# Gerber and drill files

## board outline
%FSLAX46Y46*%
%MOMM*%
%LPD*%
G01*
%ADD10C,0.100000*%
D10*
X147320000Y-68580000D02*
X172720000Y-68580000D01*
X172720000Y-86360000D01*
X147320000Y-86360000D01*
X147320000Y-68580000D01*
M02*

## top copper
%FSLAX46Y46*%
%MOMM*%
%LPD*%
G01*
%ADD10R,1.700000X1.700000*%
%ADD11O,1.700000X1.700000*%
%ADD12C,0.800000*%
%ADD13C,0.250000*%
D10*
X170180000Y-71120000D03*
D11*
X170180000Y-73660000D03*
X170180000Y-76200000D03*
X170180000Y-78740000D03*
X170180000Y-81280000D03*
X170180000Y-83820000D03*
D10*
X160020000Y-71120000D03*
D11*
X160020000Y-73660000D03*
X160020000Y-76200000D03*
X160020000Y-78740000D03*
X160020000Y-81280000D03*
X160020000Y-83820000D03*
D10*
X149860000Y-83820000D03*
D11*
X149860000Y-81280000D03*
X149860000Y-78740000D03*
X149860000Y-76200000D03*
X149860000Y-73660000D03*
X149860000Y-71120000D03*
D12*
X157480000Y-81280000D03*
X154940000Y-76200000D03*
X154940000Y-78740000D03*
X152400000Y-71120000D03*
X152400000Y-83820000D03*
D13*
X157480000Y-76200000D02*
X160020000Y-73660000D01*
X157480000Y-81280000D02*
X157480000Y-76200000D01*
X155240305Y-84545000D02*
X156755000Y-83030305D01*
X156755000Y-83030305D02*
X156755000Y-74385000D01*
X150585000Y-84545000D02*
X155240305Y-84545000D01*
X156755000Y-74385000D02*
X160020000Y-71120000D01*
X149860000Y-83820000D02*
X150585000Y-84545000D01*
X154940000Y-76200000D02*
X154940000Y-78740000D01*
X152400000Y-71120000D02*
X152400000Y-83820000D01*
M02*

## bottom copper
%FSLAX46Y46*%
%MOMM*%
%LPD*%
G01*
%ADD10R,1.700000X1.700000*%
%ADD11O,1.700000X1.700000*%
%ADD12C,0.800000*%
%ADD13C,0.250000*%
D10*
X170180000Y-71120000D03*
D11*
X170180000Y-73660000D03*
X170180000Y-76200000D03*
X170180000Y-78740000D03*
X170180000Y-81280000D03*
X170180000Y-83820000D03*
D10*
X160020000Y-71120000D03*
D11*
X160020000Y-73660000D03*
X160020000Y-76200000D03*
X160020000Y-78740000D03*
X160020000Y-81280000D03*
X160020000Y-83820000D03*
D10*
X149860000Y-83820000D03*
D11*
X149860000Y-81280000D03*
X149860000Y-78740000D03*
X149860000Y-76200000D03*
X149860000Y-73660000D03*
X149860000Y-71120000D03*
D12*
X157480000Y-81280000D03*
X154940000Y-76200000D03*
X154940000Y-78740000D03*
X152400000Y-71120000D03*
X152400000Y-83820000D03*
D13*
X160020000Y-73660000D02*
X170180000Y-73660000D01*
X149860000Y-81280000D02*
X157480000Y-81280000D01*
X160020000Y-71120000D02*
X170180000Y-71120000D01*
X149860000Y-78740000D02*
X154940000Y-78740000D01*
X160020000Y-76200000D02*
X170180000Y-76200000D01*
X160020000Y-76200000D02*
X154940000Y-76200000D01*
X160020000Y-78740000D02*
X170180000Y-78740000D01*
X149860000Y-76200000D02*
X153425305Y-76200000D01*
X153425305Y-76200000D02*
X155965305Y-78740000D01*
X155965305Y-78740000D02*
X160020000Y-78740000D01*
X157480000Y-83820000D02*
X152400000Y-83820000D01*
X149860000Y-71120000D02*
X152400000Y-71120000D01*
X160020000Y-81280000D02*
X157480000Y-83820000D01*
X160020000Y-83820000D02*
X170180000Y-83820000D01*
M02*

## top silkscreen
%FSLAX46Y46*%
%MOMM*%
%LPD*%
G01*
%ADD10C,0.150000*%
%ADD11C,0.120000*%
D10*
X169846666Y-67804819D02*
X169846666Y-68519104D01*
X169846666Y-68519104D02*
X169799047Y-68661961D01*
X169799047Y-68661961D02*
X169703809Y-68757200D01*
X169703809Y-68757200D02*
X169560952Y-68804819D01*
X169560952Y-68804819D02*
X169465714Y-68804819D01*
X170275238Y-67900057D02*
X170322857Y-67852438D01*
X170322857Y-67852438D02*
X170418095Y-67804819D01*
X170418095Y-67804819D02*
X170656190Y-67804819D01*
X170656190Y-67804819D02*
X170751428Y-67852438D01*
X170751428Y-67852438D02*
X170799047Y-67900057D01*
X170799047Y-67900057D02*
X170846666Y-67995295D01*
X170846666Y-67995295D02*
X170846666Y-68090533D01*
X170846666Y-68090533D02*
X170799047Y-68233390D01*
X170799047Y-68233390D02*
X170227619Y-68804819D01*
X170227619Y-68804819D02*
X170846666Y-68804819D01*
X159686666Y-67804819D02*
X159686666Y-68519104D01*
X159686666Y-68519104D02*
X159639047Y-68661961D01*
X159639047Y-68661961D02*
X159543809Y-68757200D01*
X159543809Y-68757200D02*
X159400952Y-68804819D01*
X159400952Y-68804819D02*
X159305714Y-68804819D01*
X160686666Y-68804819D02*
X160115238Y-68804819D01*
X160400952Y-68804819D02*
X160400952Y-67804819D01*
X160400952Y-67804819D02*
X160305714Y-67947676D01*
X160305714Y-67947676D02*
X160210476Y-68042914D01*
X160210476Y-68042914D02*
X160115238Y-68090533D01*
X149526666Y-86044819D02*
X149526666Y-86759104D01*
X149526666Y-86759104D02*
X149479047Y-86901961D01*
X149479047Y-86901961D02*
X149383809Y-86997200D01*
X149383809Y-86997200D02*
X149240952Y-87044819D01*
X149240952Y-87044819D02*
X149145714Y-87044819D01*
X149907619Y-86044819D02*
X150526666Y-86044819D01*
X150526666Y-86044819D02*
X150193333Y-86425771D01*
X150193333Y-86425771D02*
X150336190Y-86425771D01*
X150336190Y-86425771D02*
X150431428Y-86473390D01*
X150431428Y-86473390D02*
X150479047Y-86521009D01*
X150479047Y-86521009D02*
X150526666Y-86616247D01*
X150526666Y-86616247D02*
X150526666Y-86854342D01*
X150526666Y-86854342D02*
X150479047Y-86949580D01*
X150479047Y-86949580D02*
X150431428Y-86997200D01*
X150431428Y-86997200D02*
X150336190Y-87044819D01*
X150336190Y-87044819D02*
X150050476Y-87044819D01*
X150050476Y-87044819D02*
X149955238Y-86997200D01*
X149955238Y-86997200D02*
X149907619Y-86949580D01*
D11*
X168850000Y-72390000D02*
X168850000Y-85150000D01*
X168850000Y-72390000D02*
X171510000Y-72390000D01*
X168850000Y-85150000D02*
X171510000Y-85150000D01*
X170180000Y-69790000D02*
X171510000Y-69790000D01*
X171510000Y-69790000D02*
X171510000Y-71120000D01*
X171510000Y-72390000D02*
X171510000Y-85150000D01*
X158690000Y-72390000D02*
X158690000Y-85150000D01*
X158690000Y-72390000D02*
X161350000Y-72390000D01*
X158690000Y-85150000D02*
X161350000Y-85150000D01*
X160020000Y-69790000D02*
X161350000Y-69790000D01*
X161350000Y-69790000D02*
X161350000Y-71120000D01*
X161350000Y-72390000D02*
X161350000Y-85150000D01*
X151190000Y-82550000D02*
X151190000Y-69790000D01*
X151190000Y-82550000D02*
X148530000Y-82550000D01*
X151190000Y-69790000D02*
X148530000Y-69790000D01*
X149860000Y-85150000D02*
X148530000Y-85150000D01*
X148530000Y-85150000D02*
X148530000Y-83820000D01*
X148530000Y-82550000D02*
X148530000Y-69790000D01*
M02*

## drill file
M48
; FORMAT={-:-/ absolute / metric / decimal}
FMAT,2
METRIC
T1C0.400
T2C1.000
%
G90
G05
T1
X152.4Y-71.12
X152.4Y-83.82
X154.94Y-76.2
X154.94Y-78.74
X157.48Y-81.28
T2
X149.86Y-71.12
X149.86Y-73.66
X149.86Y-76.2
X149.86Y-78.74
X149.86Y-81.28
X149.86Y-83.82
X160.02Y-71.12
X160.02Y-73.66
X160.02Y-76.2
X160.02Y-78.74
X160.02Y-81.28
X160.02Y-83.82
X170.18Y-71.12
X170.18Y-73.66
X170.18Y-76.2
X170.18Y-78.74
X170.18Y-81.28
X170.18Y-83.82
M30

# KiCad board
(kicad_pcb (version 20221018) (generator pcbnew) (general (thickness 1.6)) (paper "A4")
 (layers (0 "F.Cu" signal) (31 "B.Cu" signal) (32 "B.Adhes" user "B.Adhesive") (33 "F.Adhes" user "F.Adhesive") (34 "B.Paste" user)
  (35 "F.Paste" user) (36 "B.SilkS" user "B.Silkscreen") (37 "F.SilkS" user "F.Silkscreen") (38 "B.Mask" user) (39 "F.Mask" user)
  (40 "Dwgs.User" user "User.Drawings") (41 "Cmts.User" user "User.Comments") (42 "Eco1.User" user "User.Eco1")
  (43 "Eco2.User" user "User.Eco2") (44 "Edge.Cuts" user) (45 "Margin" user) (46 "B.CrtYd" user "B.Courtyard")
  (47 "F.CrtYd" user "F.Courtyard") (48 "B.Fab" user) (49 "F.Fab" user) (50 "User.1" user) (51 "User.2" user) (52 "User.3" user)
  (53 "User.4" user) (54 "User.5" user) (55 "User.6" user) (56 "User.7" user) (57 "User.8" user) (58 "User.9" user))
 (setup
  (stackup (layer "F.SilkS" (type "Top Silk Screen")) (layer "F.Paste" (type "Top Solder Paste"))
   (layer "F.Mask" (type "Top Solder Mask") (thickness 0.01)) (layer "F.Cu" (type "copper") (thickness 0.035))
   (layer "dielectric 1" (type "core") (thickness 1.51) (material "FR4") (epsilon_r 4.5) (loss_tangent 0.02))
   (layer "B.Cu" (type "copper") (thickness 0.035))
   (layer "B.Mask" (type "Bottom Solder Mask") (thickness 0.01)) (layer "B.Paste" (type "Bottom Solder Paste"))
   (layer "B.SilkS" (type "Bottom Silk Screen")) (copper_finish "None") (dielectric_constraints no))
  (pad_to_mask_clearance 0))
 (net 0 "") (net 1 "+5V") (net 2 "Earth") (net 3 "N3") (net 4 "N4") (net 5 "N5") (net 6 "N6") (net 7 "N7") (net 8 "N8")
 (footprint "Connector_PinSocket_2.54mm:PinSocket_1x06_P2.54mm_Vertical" (layer "F.Cu") (at 170.18 71.12)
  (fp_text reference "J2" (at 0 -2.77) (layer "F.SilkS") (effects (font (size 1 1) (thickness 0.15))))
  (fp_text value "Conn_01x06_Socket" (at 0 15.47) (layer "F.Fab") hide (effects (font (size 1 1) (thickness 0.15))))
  (fp_line (start -1.33 1.27) (end -1.33 14.03) (stroke (width 0.12) (type solid)) (layer "F.SilkS"))
  (fp_line (start -1.33 1.27) (end 1.33 1.27) (stroke (width 0.12) (type solid)) (layer "F.SilkS"))
  (fp_line (start -1.33 14.03) (end 1.33 14.03) (stroke (width 0.12) (type solid)) (layer "F.SilkS"))
  (fp_line (start 0 -1.33) (end 1.33 -1.33) (stroke (width 0.12) (type solid)) (layer "F.SilkS"))
  (fp_line (start 1.33 -1.33) (end 1.33 0) (stroke (width 0.12) (type solid)) (layer "F.SilkS"))
  (fp_line (start 1.33 1.27) (end 1.33 14.03) (stroke (width 0.12) (type solid)) (layer "F.SilkS"))
  (pad "1" thru_hole rect (at 0 0) (size 1.7 1.7) (drill 1) (layers "*.Cu" "*.Mask") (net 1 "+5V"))
  (pad "2" thru_hole oval (at 0 2.54) (size 1.7 1.7) (drill 1) (layers "*.Cu" "*.Mask") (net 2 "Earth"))
  (pad "3" thru_hole oval (at 0 5.08) (size 1.7 1.7) (drill 1) (layers "*.Cu" "*.Mask") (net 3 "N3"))
  (pad "4" thru_hole oval (at 0 7.62) (size 1.7 1.7) (drill 1) (layers "*.Cu" "*.Mask") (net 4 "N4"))
  (pad "5" thru_hole oval (at 0 10.16) (size 1.7 1.7) (drill 1) (layers "*.Cu" "*.Mask") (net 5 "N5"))
  (pad "6" thru_hole oval (at 0 12.7) (size 1.7 1.7) (drill 1) (layers "*.Cu" "*.Mask") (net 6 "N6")))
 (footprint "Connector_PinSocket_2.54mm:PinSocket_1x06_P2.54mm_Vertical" (layer "F.Cu") (at 160.02 71.12)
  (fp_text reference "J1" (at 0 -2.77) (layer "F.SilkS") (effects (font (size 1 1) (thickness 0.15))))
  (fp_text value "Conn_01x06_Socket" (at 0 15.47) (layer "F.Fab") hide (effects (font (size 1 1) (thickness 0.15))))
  (fp_line (start -1.33 1.27) (end -1.33 14.03) (stroke (width 0.12) (type solid)) (layer "F.SilkS"))
  (fp_line (start -1.33 1.27) (end 1.33 1.27) (stroke (width 0.12) (type solid)) (layer "F.SilkS"))
  (fp_line (start -1.33 14.03) (end 1.33 14.03) (stroke (width 0.12) (type solid)) (layer "F.SilkS"))
  (fp_line (start 0 -1.33) (end 1.33 -1.33) (stroke (width 0.12) (type solid)) (layer "F.SilkS"))
  (fp_line (start 1.33 -1.33) (end 1.33 0) (stroke (width 0.12) (type solid)) (layer "F.SilkS"))
  (fp_line (start 1.33 1.27) (end 1.33 14.03) (stroke (width 0.12) (type solid)) (layer "F.SilkS"))
  (pad "1" thru_hole rect (at 0 0) (size 1.7 1.7) (drill 1) (layers "*.Cu" "*.Mask") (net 1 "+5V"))
  (pad "2" thru_hole oval (at 0 2.54) (size 1.7 1.7) (drill 1) (layers "*.Cu" "*.Mask") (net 2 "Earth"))
  (pad "3" thru_hole oval (at 0 5.08) (size 1.7 1.7) (drill 1) (layers "*.Cu" "*.Mask") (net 3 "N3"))
  (pad "4" thru_hole oval (at 0 7.62) (size 1.7 1.7) (drill 1) (layers "*.Cu" "*.Mask") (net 4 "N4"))
  (pad "5" thru_hole oval (at 0 10.16) (size 1.7 1.7) (drill 1) (layers "*.Cu" "*.Mask") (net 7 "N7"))
  (pad "6" thru_hole oval (at 0 12.7) (size 1.7 1.7) (drill 1) (layers "*.Cu" "*.Mask") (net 6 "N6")))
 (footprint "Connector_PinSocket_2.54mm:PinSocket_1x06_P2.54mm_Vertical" (layer "F.Cu") (at 149.86 83.82 180)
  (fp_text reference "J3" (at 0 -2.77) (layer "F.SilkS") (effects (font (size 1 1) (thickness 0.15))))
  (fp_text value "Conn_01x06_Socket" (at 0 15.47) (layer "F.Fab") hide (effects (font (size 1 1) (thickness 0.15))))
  (fp_line (start -1.33 1.27) (end -1.33 14.03) (stroke (width 0.12) (type solid)) (layer "F.SilkS"))
  (fp_line (start -1.33 1.27) (end 1.33 1.27) (stroke (width 0.12) (type solid)) (layer "F.SilkS"))
  (fp_line (start -1.33 14.03) (end 1.33 14.03) (stroke (width 0.12) (type solid)) (layer "F.SilkS"))
  (fp_line (start 0 -1.33) (end 1.33 -1.33) (stroke (width 0.12) (type solid)) (layer "F.SilkS"))
  (fp_line (start 1.33 -1.33) (end 1.33 0) (stroke (width 0.12) (type solid)) (layer "F.SilkS"))
  (fp_line (start 1.33 1.27) (end 1.33 14.03) (stroke (width 0.12) (type solid)) (layer "F.SilkS"))
  (pad "1" thru_hole rect (at 0 0 180) (size 1.7 1.7) (drill 1) (layers "*.Cu" "*.Mask") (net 1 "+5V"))
  (pad "2" thru_hole oval (at 0 2.54 180) (size 1.7 1.7) (drill 1) (layers "*.Cu" "*.Mask") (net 2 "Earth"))
  (pad "3" thru_hole oval (at 0 5.08 180) (size 1.7 1.7) (drill 1) (layers "*.Cu" "*.Mask") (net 3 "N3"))
  (pad "4" thru_hole oval (at 0 7.62 180) (size 1.7 1.7) (drill 1) (layers "*.Cu" "*.Mask") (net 4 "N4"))
  (pad "5" thru_hole oval (at 0 10.16 180) (size 1.7 1.7) (drill 1) (layers "*.Cu" "*.Mask") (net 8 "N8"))
  (pad "6" thru_hole oval (at 0 12.7 180) (size 1.7 1.7) (drill 1) (layers "*.Cu" "*.Mask") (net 7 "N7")))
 (gr_rect (start 147.32 68.58) (end 172.72 86.36) (stroke (width 0.1) (type default)) (fill none) (layer "Edge.Cuts"))
 (segment (start 157.48 76.2) (end 160.02 73.66) (width 0.25) (layer "F.Cu") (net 2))
 (segment (start 157.48 81.28) (end 157.48 76.2) (width 0.25) (layer "F.Cu") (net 2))
 (via (at 157.48 81.28) (size 0.8) (drill 0.4) (layers "F.Cu" "B.Cu") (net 2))
 (segment (start 160.02 73.66) (end 170.18 73.66) (width 0.25) (layer "B.Cu") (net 2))
 (segment (start 149.86 81.28) (end 157.48 81.28) (width 0.25) (layer "B.Cu") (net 2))
 (segment (start 155.240305 84.545) (end 156.755 83.030305) (width 0.25) (layer "F.Cu") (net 1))
 (segment (start 156.755 83.030305) (end 156.755 74.385) (width 0.25) (layer "F.Cu") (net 1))
 (segment (start 150.585 84.545) (end 155.240305 84.545) (width 0.25) (layer "F.Cu") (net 1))
 (segment (start 156.755 74.385) (end 160.02 71.12) (width 0.25) (layer "F.Cu") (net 1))
 (segment (start 149.86 83.82) (end 150.585 84.545) (width 0.25) (layer "F.Cu") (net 1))
 (segment (start 160.02 71.12) (end 170.18 71.12) (width 0.25) (layer "B.Cu") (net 1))
 (segment (start 154.94 76.2) (end 154.94 78.74) (width 0.25) (layer "F.Cu") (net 3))
 (via (at 154.94 76.2) (size 0.8) (drill 0.4) (layers "F.Cu" "B.Cu") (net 3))
 (via (at 154.94 78.74) (size 0.8) (drill 0.4) (layers "F.Cu" "B.Cu") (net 3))
 (segment (start 149.86 78.74) (end 154.94 78.74) (width 0.25) (layer "B.Cu") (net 3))
 (segment (start 160.02 76.2) (end 170.18 76.2) (width 0.25) (layer "B.Cu") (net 3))
 (segment (start 160.02 76.2) (end 154.94 76.2) (width 0.25) (layer "B.Cu") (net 3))
 (segment (start 160.02 78.74) (end 170.18 78.74) (width 0.25) (layer "B.Cu") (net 4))
 (segment (start 149.86 76.2) (end 153.425305 76.2) (width 0.25) (layer "B.Cu") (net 4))
 (segment (start 153.425305 76.2) (end 155.965305 78.74) (width 0.25) (layer "B.Cu") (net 4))
 (segment (start 155.965305 78.74) (end 160.02 78.74) (width 0.25) (layer "B.Cu") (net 4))
 (segment (start 152.4 71.12) (end 152.4 83.82) (width 0.25) (layer "F.Cu") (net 7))
 (via (at 152.4 71.12) (size 0.8) (drill 0.4) (layers "F.Cu" "B.Cu") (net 7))
 (via (at 152.4 83.82) (size 0.8) (drill 0.4) (layers "F.Cu" "B.Cu") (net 7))
 (segment (start 157.48 83.82) (end 152.4 83.82) (width 0.25) (layer "B.Cu") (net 7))
 (segment (start 149.86 71.12) (end 152.4 71.12) (width 0.25) (layer "B.Cu") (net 7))
 (segment (start 160.02 81.28) (end 157.48 83.82) (width 0.25) (layer "B.Cu") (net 7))
 (segment (start 160.02 83.82) (end 170.18 83.82) (width 0.25) (layer "B.Cu") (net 6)))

